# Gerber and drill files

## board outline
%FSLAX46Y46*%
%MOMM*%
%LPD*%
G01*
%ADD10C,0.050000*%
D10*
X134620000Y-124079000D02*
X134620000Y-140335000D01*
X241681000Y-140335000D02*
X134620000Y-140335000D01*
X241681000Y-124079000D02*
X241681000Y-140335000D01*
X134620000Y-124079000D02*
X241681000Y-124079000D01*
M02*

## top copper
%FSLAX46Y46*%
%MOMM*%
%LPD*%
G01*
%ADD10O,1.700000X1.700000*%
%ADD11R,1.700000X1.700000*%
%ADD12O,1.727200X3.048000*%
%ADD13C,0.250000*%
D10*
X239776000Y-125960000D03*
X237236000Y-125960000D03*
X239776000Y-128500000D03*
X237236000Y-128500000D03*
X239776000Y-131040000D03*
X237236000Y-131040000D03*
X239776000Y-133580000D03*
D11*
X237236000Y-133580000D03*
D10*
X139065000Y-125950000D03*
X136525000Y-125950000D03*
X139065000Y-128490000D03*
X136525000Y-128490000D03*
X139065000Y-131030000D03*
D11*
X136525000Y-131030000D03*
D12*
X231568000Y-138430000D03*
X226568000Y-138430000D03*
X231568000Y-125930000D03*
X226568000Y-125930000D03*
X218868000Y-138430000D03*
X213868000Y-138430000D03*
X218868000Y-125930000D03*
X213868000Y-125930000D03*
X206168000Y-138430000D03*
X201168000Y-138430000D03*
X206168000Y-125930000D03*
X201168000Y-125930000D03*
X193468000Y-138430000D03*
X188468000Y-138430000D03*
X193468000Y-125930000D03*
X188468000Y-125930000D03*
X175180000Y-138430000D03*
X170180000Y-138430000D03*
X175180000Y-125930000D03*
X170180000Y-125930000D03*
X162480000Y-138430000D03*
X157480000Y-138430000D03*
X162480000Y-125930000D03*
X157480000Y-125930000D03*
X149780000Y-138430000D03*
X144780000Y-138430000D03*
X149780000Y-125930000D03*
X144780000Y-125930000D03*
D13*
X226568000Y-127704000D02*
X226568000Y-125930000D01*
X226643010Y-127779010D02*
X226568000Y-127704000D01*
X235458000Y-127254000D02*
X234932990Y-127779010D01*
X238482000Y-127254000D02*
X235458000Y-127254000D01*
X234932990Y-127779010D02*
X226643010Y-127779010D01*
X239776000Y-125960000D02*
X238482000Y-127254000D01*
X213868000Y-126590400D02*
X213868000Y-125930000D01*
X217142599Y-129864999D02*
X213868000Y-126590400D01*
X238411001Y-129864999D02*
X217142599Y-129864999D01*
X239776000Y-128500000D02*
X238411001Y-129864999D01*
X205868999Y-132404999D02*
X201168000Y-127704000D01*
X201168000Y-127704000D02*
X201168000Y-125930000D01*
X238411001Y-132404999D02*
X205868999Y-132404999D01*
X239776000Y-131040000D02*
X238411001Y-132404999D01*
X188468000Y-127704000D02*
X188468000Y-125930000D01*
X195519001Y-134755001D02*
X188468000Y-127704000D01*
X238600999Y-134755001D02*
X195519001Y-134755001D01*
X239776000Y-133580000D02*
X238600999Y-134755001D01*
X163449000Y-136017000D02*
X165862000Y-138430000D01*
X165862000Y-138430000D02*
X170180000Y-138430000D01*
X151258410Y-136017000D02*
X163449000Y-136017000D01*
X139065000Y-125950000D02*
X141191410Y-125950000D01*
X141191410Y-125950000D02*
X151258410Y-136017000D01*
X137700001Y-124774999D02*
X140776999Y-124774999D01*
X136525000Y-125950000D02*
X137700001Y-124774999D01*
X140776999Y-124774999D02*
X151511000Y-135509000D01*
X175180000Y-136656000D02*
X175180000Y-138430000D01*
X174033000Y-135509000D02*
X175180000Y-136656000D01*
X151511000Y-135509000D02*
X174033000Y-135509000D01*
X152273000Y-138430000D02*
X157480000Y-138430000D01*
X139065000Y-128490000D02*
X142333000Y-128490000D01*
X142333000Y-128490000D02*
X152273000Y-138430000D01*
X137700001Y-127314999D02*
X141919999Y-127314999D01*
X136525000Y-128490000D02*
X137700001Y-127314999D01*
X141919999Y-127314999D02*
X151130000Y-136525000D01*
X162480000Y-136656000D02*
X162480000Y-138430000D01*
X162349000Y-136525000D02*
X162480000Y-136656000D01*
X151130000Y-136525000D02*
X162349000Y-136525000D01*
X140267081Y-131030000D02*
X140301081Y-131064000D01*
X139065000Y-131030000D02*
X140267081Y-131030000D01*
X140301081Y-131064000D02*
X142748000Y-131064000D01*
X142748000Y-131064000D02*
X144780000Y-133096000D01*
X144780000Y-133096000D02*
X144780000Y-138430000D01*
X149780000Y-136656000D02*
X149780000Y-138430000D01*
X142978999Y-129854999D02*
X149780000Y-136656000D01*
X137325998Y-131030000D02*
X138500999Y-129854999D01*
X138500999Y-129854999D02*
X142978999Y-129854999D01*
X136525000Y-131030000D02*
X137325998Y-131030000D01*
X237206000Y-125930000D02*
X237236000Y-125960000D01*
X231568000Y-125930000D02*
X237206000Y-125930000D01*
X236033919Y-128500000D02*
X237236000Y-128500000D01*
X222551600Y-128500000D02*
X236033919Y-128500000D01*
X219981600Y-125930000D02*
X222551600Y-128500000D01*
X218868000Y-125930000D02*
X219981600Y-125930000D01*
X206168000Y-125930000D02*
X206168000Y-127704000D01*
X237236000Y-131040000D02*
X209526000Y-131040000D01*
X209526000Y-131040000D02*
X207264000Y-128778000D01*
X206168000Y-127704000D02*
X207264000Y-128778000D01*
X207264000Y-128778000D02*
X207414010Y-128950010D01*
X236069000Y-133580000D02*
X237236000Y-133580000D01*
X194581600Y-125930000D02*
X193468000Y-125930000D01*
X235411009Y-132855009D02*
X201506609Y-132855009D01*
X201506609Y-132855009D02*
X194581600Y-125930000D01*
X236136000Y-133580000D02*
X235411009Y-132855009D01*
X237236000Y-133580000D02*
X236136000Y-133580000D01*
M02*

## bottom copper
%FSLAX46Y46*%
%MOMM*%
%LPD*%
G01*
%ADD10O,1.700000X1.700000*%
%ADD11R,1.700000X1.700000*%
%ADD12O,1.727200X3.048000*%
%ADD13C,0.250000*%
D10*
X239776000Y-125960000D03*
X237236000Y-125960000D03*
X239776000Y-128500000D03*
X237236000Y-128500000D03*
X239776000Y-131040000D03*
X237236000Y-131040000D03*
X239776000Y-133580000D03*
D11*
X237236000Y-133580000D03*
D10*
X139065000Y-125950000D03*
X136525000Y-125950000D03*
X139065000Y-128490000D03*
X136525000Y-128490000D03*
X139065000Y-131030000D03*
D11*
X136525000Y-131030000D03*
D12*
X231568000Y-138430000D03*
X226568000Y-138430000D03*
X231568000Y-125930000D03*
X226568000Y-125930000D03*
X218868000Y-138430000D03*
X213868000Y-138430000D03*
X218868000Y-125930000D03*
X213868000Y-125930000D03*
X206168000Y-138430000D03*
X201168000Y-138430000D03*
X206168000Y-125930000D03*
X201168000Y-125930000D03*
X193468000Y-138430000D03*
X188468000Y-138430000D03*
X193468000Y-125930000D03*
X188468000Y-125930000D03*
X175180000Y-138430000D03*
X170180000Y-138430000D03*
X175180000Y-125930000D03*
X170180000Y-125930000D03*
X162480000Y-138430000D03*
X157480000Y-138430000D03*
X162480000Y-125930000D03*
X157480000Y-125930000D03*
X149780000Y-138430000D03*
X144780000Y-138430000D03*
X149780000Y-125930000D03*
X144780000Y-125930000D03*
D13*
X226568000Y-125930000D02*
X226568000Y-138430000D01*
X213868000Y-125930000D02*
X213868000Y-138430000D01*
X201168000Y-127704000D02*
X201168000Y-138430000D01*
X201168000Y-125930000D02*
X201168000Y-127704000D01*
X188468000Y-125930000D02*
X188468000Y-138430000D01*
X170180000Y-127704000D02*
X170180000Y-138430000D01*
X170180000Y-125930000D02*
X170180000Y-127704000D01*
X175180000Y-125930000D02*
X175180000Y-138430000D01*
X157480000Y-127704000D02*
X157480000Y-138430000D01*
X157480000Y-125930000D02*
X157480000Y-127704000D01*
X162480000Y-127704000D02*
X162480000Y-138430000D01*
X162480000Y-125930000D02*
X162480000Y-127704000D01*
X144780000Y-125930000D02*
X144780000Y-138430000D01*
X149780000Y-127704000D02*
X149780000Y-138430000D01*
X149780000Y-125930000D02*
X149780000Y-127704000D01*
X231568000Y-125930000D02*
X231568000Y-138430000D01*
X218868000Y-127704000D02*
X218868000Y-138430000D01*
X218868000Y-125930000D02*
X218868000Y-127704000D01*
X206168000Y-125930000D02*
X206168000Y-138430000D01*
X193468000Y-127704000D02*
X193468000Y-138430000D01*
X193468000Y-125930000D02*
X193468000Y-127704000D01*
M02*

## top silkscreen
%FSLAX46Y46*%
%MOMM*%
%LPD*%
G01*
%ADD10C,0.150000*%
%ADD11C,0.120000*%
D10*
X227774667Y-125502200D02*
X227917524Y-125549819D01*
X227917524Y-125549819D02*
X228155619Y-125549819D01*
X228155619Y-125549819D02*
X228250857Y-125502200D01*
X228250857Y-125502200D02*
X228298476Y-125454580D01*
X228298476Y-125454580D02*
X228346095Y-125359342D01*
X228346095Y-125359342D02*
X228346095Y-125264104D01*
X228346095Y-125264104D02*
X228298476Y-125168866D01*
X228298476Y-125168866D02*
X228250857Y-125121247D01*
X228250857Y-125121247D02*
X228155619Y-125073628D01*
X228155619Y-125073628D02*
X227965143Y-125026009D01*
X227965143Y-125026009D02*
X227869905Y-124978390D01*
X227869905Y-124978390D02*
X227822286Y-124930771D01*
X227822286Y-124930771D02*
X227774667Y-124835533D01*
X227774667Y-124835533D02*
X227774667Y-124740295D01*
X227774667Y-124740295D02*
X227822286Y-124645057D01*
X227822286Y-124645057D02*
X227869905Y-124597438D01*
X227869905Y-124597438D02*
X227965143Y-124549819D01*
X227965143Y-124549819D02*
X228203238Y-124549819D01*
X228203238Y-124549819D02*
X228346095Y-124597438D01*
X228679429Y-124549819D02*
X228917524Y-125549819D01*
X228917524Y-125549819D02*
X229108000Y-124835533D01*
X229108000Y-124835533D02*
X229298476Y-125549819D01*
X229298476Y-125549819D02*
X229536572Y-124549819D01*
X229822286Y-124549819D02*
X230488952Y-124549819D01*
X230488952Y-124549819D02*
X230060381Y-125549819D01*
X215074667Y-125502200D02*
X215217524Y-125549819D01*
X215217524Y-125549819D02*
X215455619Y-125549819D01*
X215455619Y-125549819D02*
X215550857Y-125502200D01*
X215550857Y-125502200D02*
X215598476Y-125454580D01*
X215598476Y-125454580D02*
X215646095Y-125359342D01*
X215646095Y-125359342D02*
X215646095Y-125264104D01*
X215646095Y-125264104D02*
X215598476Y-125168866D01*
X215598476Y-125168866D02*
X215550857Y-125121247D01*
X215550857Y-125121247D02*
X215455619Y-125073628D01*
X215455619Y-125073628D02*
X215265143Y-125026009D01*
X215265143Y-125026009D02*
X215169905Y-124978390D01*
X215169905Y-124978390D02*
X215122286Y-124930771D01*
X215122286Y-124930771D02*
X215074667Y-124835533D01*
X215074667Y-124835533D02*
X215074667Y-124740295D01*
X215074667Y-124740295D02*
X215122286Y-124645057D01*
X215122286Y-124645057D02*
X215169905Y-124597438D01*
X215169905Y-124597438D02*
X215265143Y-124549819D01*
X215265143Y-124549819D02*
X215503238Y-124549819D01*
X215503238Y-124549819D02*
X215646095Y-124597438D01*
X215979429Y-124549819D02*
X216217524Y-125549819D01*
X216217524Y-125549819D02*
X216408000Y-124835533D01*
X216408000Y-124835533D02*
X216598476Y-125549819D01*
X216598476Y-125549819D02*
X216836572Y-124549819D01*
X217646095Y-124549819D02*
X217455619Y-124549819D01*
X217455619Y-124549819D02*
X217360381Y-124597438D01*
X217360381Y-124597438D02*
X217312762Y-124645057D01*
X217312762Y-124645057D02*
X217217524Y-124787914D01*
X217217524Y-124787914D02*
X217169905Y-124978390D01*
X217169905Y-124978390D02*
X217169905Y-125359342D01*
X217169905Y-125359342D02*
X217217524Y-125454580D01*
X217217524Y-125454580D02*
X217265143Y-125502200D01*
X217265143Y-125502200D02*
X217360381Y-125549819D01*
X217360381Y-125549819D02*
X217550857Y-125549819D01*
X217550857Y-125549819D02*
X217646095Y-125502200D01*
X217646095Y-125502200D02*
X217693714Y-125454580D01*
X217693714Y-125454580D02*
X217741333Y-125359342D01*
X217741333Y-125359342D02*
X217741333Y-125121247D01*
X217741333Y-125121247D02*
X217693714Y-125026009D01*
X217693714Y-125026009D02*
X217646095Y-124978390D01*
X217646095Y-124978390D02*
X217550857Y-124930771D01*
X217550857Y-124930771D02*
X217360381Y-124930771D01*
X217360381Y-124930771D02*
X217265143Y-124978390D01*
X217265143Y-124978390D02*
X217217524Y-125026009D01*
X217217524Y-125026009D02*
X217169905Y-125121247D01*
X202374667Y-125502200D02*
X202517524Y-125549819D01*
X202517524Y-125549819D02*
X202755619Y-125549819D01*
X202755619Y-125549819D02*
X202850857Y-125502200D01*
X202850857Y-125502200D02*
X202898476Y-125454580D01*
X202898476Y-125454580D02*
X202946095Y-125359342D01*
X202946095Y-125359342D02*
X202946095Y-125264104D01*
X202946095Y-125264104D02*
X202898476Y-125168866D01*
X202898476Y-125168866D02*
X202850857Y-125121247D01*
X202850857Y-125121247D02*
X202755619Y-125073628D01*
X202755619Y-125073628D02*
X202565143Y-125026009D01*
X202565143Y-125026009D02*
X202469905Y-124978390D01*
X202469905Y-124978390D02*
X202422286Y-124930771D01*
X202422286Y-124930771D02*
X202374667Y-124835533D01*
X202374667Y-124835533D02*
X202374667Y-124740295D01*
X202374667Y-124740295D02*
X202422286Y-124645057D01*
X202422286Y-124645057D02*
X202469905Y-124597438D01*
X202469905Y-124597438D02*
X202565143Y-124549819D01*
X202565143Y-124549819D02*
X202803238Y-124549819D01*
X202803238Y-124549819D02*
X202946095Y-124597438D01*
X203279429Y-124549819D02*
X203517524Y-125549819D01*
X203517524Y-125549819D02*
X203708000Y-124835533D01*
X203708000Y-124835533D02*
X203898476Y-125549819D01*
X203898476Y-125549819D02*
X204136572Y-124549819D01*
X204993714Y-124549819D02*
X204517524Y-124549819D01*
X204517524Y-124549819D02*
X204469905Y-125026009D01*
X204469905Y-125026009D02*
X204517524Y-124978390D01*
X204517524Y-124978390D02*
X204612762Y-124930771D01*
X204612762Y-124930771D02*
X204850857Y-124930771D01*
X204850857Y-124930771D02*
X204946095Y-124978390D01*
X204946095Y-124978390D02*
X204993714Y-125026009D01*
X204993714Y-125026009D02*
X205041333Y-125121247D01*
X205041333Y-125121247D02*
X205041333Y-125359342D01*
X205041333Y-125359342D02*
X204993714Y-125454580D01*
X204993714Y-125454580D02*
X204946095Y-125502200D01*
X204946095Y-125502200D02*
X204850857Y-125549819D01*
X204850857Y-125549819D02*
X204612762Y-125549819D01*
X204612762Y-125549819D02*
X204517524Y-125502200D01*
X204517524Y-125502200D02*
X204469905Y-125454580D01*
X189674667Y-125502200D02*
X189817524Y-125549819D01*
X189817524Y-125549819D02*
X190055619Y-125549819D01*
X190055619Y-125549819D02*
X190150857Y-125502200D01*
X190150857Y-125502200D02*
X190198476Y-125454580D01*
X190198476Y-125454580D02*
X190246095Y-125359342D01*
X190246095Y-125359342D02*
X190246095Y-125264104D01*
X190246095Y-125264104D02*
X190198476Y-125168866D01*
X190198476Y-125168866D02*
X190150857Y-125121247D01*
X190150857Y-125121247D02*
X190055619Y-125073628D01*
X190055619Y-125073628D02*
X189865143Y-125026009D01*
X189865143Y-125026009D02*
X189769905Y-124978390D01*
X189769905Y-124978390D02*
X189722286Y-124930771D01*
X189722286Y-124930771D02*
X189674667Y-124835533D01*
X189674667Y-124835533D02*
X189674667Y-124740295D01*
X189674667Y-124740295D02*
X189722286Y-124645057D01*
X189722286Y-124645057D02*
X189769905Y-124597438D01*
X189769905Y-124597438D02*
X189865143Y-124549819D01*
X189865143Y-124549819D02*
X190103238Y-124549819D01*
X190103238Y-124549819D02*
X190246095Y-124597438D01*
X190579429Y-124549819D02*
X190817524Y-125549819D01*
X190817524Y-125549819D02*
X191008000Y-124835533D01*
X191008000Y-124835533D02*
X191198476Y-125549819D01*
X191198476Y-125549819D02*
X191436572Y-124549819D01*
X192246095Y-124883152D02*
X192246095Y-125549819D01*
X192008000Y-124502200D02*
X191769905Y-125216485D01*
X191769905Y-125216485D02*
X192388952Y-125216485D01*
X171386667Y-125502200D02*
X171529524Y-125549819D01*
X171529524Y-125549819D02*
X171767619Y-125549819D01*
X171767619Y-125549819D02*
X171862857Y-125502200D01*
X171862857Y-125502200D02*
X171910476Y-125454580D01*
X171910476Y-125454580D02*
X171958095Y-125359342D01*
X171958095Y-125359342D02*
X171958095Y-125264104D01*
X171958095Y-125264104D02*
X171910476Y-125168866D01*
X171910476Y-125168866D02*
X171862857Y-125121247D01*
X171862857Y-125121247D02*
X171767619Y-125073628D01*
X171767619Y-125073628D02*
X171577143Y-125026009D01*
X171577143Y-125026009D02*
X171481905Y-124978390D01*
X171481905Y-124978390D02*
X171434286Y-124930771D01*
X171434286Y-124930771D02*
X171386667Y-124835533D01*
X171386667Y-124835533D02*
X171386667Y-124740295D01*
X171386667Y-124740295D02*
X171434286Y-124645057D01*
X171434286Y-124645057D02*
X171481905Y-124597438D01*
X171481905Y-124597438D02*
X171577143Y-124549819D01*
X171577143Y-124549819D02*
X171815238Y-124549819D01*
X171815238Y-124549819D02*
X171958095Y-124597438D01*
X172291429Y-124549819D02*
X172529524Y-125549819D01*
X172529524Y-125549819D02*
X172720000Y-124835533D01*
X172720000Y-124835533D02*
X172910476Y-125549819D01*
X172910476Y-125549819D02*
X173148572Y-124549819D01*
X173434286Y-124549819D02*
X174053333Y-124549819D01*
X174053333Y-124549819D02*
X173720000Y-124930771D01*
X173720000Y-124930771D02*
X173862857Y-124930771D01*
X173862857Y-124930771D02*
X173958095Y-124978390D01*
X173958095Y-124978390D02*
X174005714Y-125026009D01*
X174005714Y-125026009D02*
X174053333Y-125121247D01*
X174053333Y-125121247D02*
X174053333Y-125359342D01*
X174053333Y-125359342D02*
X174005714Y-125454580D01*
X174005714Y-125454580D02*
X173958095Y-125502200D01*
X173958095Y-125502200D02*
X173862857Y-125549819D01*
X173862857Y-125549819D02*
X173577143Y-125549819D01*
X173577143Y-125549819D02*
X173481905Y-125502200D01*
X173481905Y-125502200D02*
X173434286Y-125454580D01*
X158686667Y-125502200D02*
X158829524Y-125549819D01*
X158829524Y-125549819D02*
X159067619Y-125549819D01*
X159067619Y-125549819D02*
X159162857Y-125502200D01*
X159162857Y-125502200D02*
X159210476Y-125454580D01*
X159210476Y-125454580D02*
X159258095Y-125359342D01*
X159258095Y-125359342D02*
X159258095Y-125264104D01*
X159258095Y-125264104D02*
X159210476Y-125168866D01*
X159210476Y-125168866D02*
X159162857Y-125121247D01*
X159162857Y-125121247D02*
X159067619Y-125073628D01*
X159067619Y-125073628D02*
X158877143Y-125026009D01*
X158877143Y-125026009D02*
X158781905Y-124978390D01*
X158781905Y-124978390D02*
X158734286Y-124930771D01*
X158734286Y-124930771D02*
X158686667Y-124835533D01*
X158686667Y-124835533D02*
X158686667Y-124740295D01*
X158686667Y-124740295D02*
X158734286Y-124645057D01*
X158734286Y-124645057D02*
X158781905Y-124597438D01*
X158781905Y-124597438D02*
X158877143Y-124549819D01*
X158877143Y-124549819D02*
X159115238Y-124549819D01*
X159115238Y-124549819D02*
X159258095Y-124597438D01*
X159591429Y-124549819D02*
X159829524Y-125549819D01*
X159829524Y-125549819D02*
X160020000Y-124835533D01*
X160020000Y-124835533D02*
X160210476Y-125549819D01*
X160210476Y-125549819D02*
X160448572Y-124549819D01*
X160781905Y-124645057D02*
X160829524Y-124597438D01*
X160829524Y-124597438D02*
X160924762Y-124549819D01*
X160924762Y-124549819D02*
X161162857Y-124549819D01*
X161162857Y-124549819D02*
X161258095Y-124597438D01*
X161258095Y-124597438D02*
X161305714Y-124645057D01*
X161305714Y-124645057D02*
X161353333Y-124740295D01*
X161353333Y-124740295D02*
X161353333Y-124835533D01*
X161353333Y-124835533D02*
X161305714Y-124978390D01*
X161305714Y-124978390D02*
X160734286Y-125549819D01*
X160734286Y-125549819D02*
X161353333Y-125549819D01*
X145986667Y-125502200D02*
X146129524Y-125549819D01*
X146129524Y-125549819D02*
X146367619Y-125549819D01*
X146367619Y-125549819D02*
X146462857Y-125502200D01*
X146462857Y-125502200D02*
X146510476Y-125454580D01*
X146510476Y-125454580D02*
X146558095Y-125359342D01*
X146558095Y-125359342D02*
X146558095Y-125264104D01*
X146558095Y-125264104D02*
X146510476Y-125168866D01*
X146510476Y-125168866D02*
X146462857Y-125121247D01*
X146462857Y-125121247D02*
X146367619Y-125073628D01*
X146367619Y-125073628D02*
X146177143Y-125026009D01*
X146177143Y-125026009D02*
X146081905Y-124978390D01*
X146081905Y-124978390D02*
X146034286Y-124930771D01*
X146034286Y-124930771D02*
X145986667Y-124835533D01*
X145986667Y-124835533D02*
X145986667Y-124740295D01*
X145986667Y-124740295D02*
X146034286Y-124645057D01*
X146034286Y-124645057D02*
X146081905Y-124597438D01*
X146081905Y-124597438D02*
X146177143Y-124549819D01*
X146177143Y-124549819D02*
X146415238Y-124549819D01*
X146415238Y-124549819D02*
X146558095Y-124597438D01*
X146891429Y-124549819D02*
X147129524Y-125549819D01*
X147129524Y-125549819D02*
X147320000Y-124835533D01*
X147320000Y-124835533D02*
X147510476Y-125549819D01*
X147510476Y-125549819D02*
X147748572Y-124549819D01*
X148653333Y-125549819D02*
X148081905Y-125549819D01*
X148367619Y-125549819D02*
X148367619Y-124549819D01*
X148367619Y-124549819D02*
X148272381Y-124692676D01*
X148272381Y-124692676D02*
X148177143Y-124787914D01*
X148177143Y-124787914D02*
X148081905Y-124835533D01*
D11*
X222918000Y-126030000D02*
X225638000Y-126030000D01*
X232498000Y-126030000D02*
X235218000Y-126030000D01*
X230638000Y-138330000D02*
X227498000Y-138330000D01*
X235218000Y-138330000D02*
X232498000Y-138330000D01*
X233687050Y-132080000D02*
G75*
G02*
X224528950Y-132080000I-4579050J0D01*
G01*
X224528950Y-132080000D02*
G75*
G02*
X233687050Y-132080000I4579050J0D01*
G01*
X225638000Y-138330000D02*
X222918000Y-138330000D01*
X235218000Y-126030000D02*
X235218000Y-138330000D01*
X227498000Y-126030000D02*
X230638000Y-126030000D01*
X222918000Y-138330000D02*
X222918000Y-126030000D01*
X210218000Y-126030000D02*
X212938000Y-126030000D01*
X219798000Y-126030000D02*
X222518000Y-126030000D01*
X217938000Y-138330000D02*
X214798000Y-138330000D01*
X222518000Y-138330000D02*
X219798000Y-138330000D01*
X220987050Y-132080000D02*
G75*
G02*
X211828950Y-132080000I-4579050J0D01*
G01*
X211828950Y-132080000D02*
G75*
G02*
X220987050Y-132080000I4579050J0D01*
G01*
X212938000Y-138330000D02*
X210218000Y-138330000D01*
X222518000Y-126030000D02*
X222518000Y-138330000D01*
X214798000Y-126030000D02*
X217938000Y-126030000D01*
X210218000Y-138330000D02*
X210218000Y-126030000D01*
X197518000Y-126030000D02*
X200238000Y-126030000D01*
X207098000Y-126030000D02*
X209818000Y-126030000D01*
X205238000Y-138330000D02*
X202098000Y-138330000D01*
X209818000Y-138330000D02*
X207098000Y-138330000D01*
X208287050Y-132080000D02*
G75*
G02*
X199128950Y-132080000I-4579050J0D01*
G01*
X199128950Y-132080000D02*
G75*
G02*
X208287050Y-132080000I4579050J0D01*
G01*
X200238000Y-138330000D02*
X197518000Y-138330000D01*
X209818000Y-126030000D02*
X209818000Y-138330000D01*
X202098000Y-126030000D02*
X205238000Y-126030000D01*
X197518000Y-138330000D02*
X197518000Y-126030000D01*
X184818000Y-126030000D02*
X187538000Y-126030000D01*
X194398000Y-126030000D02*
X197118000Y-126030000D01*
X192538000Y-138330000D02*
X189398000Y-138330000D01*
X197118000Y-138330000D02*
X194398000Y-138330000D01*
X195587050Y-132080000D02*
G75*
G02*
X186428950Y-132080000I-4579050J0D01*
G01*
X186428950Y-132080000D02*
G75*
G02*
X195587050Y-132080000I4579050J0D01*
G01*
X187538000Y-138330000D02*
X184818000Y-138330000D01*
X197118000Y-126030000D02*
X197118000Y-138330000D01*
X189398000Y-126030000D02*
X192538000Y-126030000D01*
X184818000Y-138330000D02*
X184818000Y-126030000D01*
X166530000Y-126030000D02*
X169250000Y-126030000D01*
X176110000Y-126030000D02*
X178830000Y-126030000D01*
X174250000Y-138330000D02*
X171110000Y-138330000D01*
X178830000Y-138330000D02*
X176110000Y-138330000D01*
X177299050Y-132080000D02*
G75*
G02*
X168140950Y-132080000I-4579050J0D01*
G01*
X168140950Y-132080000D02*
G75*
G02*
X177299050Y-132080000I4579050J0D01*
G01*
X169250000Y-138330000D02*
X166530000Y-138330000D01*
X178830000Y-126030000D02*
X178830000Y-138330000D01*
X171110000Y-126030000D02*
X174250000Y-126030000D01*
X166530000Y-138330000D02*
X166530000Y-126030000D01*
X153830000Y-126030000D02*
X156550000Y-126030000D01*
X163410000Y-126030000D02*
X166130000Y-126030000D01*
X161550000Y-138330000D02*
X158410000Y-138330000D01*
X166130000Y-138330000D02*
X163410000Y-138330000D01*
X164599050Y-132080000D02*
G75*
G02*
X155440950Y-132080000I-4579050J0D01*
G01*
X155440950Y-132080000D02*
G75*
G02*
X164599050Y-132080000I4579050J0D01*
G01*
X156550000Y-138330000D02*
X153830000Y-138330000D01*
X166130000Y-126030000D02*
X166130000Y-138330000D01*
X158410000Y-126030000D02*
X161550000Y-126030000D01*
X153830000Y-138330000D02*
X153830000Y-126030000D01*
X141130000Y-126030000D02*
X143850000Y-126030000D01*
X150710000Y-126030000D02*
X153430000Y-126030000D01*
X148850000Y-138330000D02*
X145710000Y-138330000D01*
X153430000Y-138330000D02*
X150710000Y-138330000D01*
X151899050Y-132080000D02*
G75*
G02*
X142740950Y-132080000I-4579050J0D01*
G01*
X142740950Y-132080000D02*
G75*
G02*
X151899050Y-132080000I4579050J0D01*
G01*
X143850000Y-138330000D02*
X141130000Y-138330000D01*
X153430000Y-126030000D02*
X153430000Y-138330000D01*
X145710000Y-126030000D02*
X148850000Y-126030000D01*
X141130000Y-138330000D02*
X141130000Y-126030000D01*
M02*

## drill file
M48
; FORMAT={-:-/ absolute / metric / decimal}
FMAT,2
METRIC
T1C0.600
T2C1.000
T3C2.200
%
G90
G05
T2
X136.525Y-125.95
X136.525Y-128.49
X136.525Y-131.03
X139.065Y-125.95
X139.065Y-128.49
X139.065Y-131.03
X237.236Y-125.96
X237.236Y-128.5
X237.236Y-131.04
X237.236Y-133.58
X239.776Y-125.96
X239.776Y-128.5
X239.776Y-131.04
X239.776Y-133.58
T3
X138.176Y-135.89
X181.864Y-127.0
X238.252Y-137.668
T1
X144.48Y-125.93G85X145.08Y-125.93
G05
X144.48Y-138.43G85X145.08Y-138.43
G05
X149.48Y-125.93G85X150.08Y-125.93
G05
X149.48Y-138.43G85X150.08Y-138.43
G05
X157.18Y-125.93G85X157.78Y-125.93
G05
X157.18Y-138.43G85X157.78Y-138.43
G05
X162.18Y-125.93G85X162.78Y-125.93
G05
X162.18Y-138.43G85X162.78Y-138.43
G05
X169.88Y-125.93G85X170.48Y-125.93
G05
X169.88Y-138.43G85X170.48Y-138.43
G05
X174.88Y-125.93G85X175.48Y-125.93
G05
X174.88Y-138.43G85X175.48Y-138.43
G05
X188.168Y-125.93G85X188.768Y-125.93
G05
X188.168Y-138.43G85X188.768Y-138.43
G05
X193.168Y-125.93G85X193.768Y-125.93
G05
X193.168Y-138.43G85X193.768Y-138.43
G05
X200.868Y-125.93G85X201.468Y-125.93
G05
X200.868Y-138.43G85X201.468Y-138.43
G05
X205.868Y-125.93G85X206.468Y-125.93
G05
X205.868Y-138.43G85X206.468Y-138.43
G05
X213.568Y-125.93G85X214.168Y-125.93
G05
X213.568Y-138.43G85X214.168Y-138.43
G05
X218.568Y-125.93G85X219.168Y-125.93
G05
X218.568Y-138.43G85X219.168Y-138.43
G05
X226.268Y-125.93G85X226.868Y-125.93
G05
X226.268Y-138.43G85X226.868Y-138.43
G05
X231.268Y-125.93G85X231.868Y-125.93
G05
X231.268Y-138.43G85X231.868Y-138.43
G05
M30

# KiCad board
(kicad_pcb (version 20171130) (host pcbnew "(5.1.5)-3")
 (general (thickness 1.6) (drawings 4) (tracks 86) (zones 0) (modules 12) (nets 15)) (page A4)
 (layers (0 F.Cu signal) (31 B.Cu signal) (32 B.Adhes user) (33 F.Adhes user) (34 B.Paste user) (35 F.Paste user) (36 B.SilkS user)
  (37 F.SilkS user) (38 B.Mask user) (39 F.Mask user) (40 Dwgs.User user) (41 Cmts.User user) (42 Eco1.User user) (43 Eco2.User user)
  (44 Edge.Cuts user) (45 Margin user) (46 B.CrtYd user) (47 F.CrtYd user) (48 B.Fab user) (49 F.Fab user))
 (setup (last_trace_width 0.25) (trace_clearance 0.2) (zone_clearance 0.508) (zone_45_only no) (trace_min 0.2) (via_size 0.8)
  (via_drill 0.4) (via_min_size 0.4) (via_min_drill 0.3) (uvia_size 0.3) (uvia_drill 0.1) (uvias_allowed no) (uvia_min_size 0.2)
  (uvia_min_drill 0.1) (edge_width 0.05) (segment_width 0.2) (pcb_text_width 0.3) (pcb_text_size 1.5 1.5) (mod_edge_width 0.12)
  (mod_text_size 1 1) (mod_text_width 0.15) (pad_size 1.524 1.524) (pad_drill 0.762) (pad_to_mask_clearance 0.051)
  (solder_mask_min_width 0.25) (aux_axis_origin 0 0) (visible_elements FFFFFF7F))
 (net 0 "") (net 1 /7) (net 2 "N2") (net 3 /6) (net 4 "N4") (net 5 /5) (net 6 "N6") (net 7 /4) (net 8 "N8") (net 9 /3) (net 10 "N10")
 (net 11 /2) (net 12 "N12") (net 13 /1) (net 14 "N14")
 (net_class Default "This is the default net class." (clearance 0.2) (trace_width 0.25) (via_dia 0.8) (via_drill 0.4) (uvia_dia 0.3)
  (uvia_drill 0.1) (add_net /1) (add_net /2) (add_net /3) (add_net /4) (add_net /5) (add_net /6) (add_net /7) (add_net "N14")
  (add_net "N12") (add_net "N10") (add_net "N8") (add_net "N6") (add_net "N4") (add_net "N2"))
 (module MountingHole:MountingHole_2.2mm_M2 (layer F.Cu) (at 181.864 127)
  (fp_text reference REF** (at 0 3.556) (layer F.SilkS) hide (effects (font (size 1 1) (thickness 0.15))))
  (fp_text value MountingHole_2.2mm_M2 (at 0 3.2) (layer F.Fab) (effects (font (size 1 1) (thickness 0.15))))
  (pad 1 np_thru_hole circle (at 0 0) (size 2.2 2.2) (drill 2.2) (layers *.Cu *.Mask)))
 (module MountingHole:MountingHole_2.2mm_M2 (layer F.Cu) (at 238.252 137.668)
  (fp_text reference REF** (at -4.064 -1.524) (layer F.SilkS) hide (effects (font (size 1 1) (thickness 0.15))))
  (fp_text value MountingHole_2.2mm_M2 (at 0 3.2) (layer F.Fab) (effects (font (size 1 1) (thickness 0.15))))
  (pad 1 np_thru_hole circle (at 0 0) (size 2.2 2.2) (drill 2.2) (layers *.Cu *.Mask)))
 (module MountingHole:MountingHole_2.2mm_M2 (layer F.Cu) (at 138.176 135.89)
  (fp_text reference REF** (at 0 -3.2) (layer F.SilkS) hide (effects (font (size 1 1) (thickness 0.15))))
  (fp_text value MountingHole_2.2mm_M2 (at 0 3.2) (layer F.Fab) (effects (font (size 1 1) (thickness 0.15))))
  (pad 1 np_thru_hole circle (at 0 0) (size 2.2 2.2) (drill 2.2) (layers *.Cu *.Mask)))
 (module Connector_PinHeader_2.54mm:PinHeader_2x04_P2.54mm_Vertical (layer B.Cu) (at 237.236 133.58)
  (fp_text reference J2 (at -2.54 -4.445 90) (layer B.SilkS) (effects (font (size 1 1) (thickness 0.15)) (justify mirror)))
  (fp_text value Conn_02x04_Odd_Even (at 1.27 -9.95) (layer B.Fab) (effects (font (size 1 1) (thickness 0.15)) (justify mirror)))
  (pad 8 thru_hole oval (at 2.54 -7.62) (size 1.7 1.7) (drill 1) (layers *.Cu *.Mask) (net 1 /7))
  (pad 7 thru_hole oval (at 0 -7.62) (size 1.7 1.7) (drill 1) (layers *.Cu *.Mask) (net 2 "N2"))
  (pad 6 thru_hole oval (at 2.54 -5.08) (size 1.7 1.7) (drill 1) (layers *.Cu *.Mask) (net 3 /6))
  (pad 5 thru_hole oval (at 0 -5.08) (size 1.7 1.7) (drill 1) (layers *.Cu *.Mask) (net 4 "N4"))
  (pad 4 thru_hole oval (at 2.54 -2.54) (size 1.7 1.7) (drill 1) (layers *.Cu *.Mask) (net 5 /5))
  (pad 3 thru_hole oval (at 0 -2.54) (size 1.7 1.7) (drill 1) (layers *.Cu *.Mask) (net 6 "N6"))
  (pad 2 thru_hole oval (at 2.54 0) (size 1.7 1.7) (drill 1) (layers *.Cu *.Mask) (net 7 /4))
  (pad 1 thru_hole rect (at 0 0) (size 1.7 1.7) (drill 1) (layers *.Cu *.Mask) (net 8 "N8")))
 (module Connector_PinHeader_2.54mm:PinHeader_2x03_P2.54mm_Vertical (layer B.Cu) (at 136.525 131.03)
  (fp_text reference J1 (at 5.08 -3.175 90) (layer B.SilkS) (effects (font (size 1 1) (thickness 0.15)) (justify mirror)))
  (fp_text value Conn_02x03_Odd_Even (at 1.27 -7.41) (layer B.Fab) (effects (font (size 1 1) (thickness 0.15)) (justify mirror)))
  (pad 6 thru_hole oval (at 2.54 -5.08) (size 1.7 1.7) (drill 1) (layers *.Cu *.Mask) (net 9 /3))
  (pad 5 thru_hole oval (at 0 -5.08) (size 1.7 1.7) (drill 1) (layers *.Cu *.Mask) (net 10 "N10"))
  (pad 4 thru_hole oval (at 2.54 -2.54) (size 1.7 1.7) (drill 1) (layers *.Cu *.Mask) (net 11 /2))
  (pad 3 thru_hole oval (at 0 -2.54) (size 1.7 1.7) (drill 1) (layers *.Cu *.Mask) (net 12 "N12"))
  (pad 2 thru_hole oval (at 2.54 0) (size 1.7 1.7) (drill 1) (layers *.Cu *.Mask) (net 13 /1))
  (pad 1 thru_hole rect (at 0 0) (size 1.7 1.7) (drill 1) (layers *.Cu *.Mask) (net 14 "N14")))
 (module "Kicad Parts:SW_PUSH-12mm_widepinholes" (layer F.Cu) (at 226.568 138.43 90)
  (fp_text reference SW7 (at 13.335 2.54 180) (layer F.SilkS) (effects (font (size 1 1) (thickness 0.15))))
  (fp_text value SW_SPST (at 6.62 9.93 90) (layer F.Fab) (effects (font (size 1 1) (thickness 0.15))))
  (fp_line (start 12.4 -3.65) (end 12.4 -0.93) (layer F.SilkS) (width 0.12))
  (fp_line (start 12.4 5.93) (end 12.4 8.65) (layer F.SilkS) (width 0.12))
  (fp_line (start 0.1 4.07) (end 0.1 0.93) (layer F.SilkS) (width 0.12))
  (fp_line (start 0.1 8.65) (end 0.1 5.93) (layer F.SilkS) (width 0.12))
  (fp_circle (center 6.35 2.54) (end 10.16 5.08) (layer F.SilkS) (width 0.12))
  (fp_line (start 0.1 -0.93) (end 0.1 -3.65) (layer F.SilkS) (width 0.12))
  (fp_line (start 12.4 8.65) (end 0.1 8.65) (layer F.SilkS) (width 0.12))
  (fp_line (start 12.4 0.93) (end 12.4 4.07) (layer F.SilkS) (width 0.12))
  (fp_line (start 0.1 -3.65) (end 12.4 -3.65) (layer F.SilkS) (width 0.12))
  (pad 2 thru_hole oval (at 0 5 90) (size 3.048 1.7272) (drill oval 0.6 1.2) (layers *.Cu *.Mask) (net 2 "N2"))
  (pad 1 thru_hole oval (at 0 0 90) (size 3.048 1.7272) (drill oval 0.6 1.2) (layers *.Cu *.Mask) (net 1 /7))
  (pad 2 thru_hole oval (at 12.5 5 90) (size 3.048 1.7272) (drill oval 0.6 1.2) (layers *.Cu *.Mask) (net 2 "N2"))
  (pad 1 thru_hole oval (at 12.5 0 90) (size 3.048 1.7272) (drill oval 0.6 1.2) (layers *.Cu *.Mask) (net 1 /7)))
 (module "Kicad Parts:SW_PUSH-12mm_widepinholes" (layer F.Cu) (at 213.868 138.43 90)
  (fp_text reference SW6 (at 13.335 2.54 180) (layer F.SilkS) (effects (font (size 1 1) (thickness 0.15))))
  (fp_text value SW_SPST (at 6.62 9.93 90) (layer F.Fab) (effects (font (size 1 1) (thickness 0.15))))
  (fp_line (start 12.4 -3.65) (end 12.4 -0.93) (layer F.SilkS) (width 0.12))
  (fp_line (start 12.4 5.93) (end 12.4 8.65) (layer F.SilkS) (width 0.12))
  (fp_line (start 0.1 4.07) (end 0.1 0.93) (layer F.SilkS) (width 0.12))
  (fp_line (start 0.1 8.65) (end 0.1 5.93) (layer F.SilkS) (width 0.12))
  (fp_circle (center 6.35 2.54) (end 10.16 5.08) (layer F.SilkS) (width 0.12))
  (fp_line (start 0.1 -0.93) (end 0.1 -3.65) (layer F.SilkS) (width 0.12))
  (fp_line (start 12.4 8.65) (end 0.1 8.65) (layer F.SilkS) (width 0.12))
  (fp_line (start 12.4 0.93) (end 12.4 4.07) (layer F.SilkS) (width 0.12))
  (fp_line (start 0.1 -3.65) (end 12.4 -3.65) (layer F.SilkS) (width 0.12))
  (pad 2 thru_hole oval (at 0 5 90) (size 3.048 1.7272) (drill oval 0.6 1.2) (layers *.Cu *.Mask) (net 4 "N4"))
  (pad 1 thru_hole oval (at 0 0 90) (size 3.048 1.7272) (drill oval 0.6 1.2) (layers *.Cu *.Mask) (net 3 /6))
  (pad 2 thru_hole oval (at 12.5 5 90) (size 3.048 1.7272) (drill oval 0.6 1.2) (layers *.Cu *.Mask) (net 4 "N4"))
  (pad 1 thru_hole oval (at 12.5 0 90) (size 3.048 1.7272) (drill oval 0.6 1.2) (layers *.Cu *.Mask) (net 3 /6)))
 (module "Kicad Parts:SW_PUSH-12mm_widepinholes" (layer F.Cu) (at 201.168 138.43 90)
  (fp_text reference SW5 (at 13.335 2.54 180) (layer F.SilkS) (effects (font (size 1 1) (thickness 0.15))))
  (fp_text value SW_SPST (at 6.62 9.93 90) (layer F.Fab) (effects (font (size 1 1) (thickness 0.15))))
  (fp_line (start 12.4 -3.65) (end 12.4 -0.93) (layer F.SilkS) (width 0.12))
  (fp_line (start 12.4 5.93) (end 12.4 8.65) (layer F.SilkS) (width 0.12))
  (fp_line (start 0.1 4.07) (end 0.1 0.93) (layer F.SilkS) (width 0.12))
  (fp_line (start 0.1 8.65) (end 0.1 5.93) (layer F.SilkS) (width 0.12))
  (fp_circle (center 6.35 2.54) (end 10.16 5.08) (layer F.SilkS) (width 0.12))
  (fp_line (start 0.1 -0.93) (end 0.1 -3.65) (layer F.SilkS) (width 0.12))
  (fp_line (start 12.4 8.65) (end 0.1 8.65) (layer F.SilkS) (width 0.12))
  (fp_line (start 12.4 0.93) (end 12.4 4.07) (layer F.SilkS) (width 0.12))
  (fp_line (start 0.1 -3.65) (end 12.4 -3.65) (layer F.SilkS) (width 0.12))
  (pad 2 thru_hole oval (at 0 5 90) (size 3.048 1.7272) (drill oval 0.6 1.2) (layers *.Cu *.Mask) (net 6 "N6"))
  (pad 1 thru_hole oval (at 0 0 90) (size 3.048 1.7272) (drill oval 0.6 1.2) (layers *.Cu *.Mask) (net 5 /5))
  (pad 2 thru_hole oval (at 12.5 5 90) (size 3.048 1.7272) (drill oval 0.6 1.2) (layers *.Cu *.Mask) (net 6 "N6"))
  (pad 1 thru_hole oval (at 12.5 0 90) (size 3.048 1.7272) (drill oval 0.6 1.2) (layers *.Cu *.Mask) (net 5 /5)))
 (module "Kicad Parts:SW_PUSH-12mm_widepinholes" (layer F.Cu) (at 188.468 138.43 90)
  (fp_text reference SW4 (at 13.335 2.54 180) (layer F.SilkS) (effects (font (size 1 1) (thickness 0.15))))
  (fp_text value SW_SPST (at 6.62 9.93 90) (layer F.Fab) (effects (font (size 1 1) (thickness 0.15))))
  (fp_line (start 12.4 -3.65) (end 12.4 -0.93) (layer F.SilkS) (width 0.12))
  (fp_line (start 12.4 5.93) (end 12.4 8.65) (layer F.SilkS) (width 0.12))
  (fp_line (start 0.1 4.07) (end 0.1 0.93) (layer F.SilkS) (width 0.12))
  (fp_line (start 0.1 8.65) (end 0.1 5.93) (layer F.SilkS) (width 0.12))
  (fp_circle (center 6.35 2.54) (end 10.16 5.08) (layer F.SilkS) (width 0.12))
  (fp_line (start 0.1 -0.93) (end 0.1 -3.65) (layer F.SilkS) (width 0.12))
  (fp_line (start 12.4 8.65) (end 0.1 8.65) (layer F.SilkS) (width 0.12))
  (fp_line (start 12.4 0.93) (end 12.4 4.07) (layer F.SilkS) (width 0.12))
  (fp_line (start 0.1 -3.65) (end 12.4 -3.65) (layer F.SilkS) (width 0.12))
  (pad 2 thru_hole oval (at 0 5 90) (size 3.048 1.7272) (drill oval 0.6 1.2) (layers *.Cu *.Mask) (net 8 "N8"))
  (pad 1 thru_hole oval (at 0 0 90) (size 3.048 1.7272) (drill oval 0.6 1.2) (layers *.Cu *.Mask) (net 7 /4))
  (pad 2 thru_hole oval (at 12.5 5 90) (size 3.048 1.7272) (drill oval 0.6 1.2) (layers *.Cu *.Mask) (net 8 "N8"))
  (pad 1 thru_hole oval (at 12.5 0 90) (size 3.048 1.7272) (drill oval 0.6 1.2) (layers *.Cu *.Mask) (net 7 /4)))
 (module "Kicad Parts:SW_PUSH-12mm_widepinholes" (layer F.Cu) (at 170.18 138.43 90)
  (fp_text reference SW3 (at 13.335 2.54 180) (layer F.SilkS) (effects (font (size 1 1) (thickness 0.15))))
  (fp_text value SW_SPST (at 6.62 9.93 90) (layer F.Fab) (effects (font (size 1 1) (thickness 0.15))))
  (fp_line (start 12.4 -3.65) (end 12.4 -0.93) (layer F.SilkS) (width 0.12))
  (fp_line (start 12.4 5.93) (end 12.4 8.65) (layer F.SilkS) (width 0.12))
  (fp_line (start 0.1 4.07) (end 0.1 0.93) (layer F.SilkS) (width 0.12))
  (fp_line (start 0.1 8.65) (end 0.1 5.93) (layer F.SilkS) (width 0.12))
  (fp_circle (center 6.35 2.54) (end 10.16 5.08) (layer F.SilkS) (width 0.12))
  (fp_line (start 0.1 -0.93) (end 0.1 -3.65) (layer F.SilkS) (width 0.12))
  (fp_line (start 12.4 8.65) (end 0.1 8.65) (layer F.SilkS) (width 0.12))
  (fp_line (start 12.4 0.93) (end 12.4 4.07) (layer F.SilkS) (width 0.12))
  (fp_line (start 0.1 -3.65) (end 12.4 -3.65) (layer F.SilkS) (width 0.12))
  (pad 2 thru_hole oval (at 0 5 90) (size 3.048 1.7272) (drill oval 0.6 1.2) (layers *.Cu *.Mask) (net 10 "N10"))
  (pad 1 thru_hole oval (at 0 0 90) (size 3.048 1.7272) (drill oval 0.6 1.2) (layers *.Cu *.Mask) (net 9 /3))
  (pad 2 thru_hole oval (at 12.5 5 90) (size 3.048 1.7272) (drill oval 0.6 1.2) (layers *.Cu *.Mask) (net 10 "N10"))
  (pad 1 thru_hole oval (at 12.5 0 90) (size 3.048 1.7272) (drill oval 0.6 1.2) (layers *.Cu *.Mask) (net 9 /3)))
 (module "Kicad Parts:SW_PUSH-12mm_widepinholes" (layer F.Cu) (at 157.48 138.43 90)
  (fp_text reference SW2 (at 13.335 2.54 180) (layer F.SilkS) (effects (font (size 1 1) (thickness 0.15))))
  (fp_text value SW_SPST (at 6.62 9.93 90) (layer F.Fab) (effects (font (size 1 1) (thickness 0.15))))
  (fp_line (start 12.4 -3.65) (end 12.4 -0.93) (layer F.SilkS) (width 0.12))
  (fp_line (start 12.4 5.93) (end 12.4 8.65) (layer F.SilkS) (width 0.12))
  (fp_line (start 0.1 4.07) (end 0.1 0.93) (layer F.SilkS) (width 0.12))
  (fp_line (start 0.1 8.65) (end 0.1 5.93) (layer F.SilkS) (width 0.12))
  (fp_circle (center 6.35 2.54) (end 10.16 5.08) (layer F.SilkS) (width 0.12))
  (fp_line (start 0.1 -0.93) (end 0.1 -3.65) (layer F.SilkS) (width 0.12))
  (fp_line (start 12.4 8.65) (end 0.1 8.65) (layer F.SilkS) (width 0.12))
  (fp_line (start 12.4 0.93) (end 12.4 4.07) (layer F.SilkS) (width 0.12))
  (fp_line (start 0.1 -3.65) (end 12.4 -3.65) (layer F.SilkS) (width 0.12))
  (pad 2 thru_hole oval (at 0 5 90) (size 3.048 1.7272) (drill oval 0.6 1.2) (layers *.Cu *.Mask) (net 12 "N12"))
  (pad 1 thru_hole oval (at 0 0 90) (size 3.048 1.7272) (drill oval 0.6 1.2) (layers *.Cu *.Mask) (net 11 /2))
  (pad 2 thru_hole oval (at 12.5 5 90) (size 3.048 1.7272) (drill oval 0.6 1.2) (layers *.Cu *.Mask) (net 12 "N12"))
  (pad 1 thru_hole oval (at 12.5 0 90) (size 3.048 1.7272) (drill oval 0.6 1.2) (layers *.Cu *.Mask) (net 11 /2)))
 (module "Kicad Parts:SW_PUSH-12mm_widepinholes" (layer F.Cu) (at 144.78 138.43 90)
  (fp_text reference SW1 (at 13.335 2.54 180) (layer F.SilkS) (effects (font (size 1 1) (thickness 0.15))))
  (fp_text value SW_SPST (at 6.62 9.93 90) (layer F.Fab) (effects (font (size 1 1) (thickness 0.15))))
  (fp_line (start 12.4 -3.65) (end 12.4 -0.93) (layer F.SilkS) (width 0.12))
  (fp_line (start 12.4 5.93) (end 12.4 8.65) (layer F.SilkS) (width 0.12))
  (fp_line (start 0.1 4.07) (end 0.1 0.93) (layer F.SilkS) (width 0.12))
  (fp_line (start 0.1 8.65) (end 0.1 5.93) (layer F.SilkS) (width 0.12))
  (fp_circle (center 6.35 2.54) (end 10.16 5.08) (layer F.SilkS) (width 0.12))
  (fp_line (start 0.1 -0.93) (end 0.1 -3.65) (layer F.SilkS) (width 0.12))
  (fp_line (start 12.4 8.65) (end 0.1 8.65) (layer F.SilkS) (width 0.12))
  (fp_line (start 12.4 0.93) (end 12.4 4.07) (layer F.SilkS) (width 0.12))
  (fp_line (start 0.1 -3.65) (end 12.4 -3.65) (layer F.SilkS) (width 0.12))
  (pad 2 thru_hole oval (at 0 5 90) (size 3.048 1.7272) (drill oval 0.6 1.2) (layers *.Cu *.Mask) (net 14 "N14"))
  (pad 1 thru_hole oval (at 0 0 90) (size 3.048 1.7272) (drill oval 0.6 1.2) (layers *.Cu *.Mask) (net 13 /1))
  (pad 2 thru_hole oval (at 12.5 5 90) (size 3.048 1.7272) (drill oval 0.6 1.2) (layers *.Cu *.Mask) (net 14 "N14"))
  (pad 1 thru_hole oval (at 12.5 0 90) (size 3.048 1.7272) (drill oval 0.6 1.2) (layers *.Cu *.Mask) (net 13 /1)))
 (gr_line (start 134.62 124.079) (end 134.62 140.335) (layer Edge.Cuts) (width 0.05))
 (gr_line (start 241.681 140.335) (end 134.62 140.335) (layer Edge.Cuts) (width 0.05))
 (gr_line (start 241.681 124.079) (end 241.681 140.335) (layer Edge.Cuts) (width 0.05))
 (gr_line (start 134.62 124.079) (end 241.681 124.079) (layer Edge.Cuts) (width 0.05))
 (segment (start 226.568 125.93) (end 226.568 138.43) (width 0.25) (layer B.Cu) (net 1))
 (segment (start 226.568 127.704) (end 226.568 125.93) (width 0.25) (layer F.Cu) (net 1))
 (segment (start 226.64301 127.77901) (end 226.568 127.704) (width 0.25) (layer F.Cu) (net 1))
 (segment (start 235.458 127.254) (end 234.93299 127.77901) (width 0.25) (layer F.Cu) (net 1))
 (segment (start 238.482 127.254) (end 235.458 127.254) (width 0.25) (layer F.Cu) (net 1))
 (segment (start 234.93299 127.77901) (end 226.64301 127.77901) (width 0.25) (layer F.Cu) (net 1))
 (segment (start 239.776 125.96) (end 238.482 127.254) (width 0.25) (layer F.Cu) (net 1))
 (segment (start 213.868 125.93) (end 213.868 138.43) (width 0.25) (layer B.Cu) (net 3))
 (segment (start 213.868 126.5904) (end 213.868 125.93) (width 0.25) (layer F.Cu) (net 3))
 (segment (start 217.142599 129.864999) (end 213.868 126.5904) (width 0.25) (layer F.Cu) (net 3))
 (segment (start 238.411001 129.864999) (end 217.142599 129.864999) (width 0.25) (layer F.Cu) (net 3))
 (segment (start 239.776 128.5) (end 238.411001 129.864999) (width 0.25) (layer F.Cu) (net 3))
 (segment (start 201.168 127.704) (end 201.168 138.43) (width 0.25) (layer B.Cu) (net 5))
 (segment (start 201.168 125.93) (end 201.168 127.704) (width 0.25) (layer B.Cu) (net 5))
 (segment (start 205.868999 132.404999) (end 201.168 127.704) (width 0.25) (layer F.Cu) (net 5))
 (segment (start 201.168 127.704) (end 201.168 125.93) (width 0.25) (layer F.Cu) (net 5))
 (segment (start 238.411001 132.404999) (end 205.868999 132.404999) (width 0.25) (layer F.Cu) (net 5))
 (segment (start 239.776 131.04) (end 238.411001 132.404999) (width 0.25) (layer F.Cu) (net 5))
 (segment (start 188.468 125.93) (end 188.468 138.43) (width 0.25) (layer B.Cu) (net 7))
 (segment (start 188.468 127.704) (end 188.468 125.93) (width 0.25) (layer F.Cu) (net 7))
 (segment (start 195.519001 134.755001) (end 188.468 127.704) (width 0.25) (layer F.Cu) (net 7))
 (segment (start 238.600999 134.755001) (end 195.519001 134.755001) (width 0.25) (layer F.Cu) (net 7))
 (segment (start 239.776 133.58) (end 238.600999 134.755001) (width 0.25) (layer F.Cu) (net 7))
 (segment (start 170.18 127.704) (end 170.18 138.43) (width 0.25) (layer B.Cu) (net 9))
 (segment (start 170.18 125.93) (end 170.18 127.704) (width 0.25) (layer B.Cu) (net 9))
 (segment (start 163.449 136.017) (end 165.862 138.43) (width 0.25) (layer F.Cu) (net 9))
 (segment (start 165.862 138.43) (end 170.18 138.43) (width 0.25) (layer F.Cu) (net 9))
 (segment (start 151.25841 136.017) (end 163.449 136.017) (width 0.25) (layer F.Cu) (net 9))
 (segment (start 139.065 125.95) (end 141.19141 125.95) (width 0.25) (layer F.Cu) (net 9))
 (segment (start 141.19141 125.95) (end 151.25841 136.017) (width 0.25) (layer F.Cu) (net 9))
 (segment (start 175.18 125.93) (end 175.18 138.43) (width 0.25) (layer B.Cu) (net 10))
 (segment (start 137.700001 124.774999) (end 140.776999 124.774999) (width 0.25) (layer F.Cu) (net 10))
 (segment (start 136.525 125.95) (end 137.700001 124.774999) (width 0.25) (layer F.Cu) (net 10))
 (segment (start 140.776999 124.774999) (end 151.511 135.509) (width 0.25) (layer F.Cu) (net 10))
 (segment (start 175.18 136.656) (end 175.18 138.43) (width 0.25) (layer F.Cu) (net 10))
 (segment (start 174.033 135.509) (end 175.18 136.656) (width 0.25) (layer F.Cu) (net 10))
 (segment (start 151.511 135.509) (end 174.033 135.509) (width 0.25) (layer F.Cu) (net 10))
 (segment (start 157.48 127.704) (end 157.48 138.43) (width 0.25) (layer B.Cu) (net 11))
 (segment (start 157.48 125.93) (end 157.48 127.704) (width 0.25) (layer B.Cu) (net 11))
 (segment (start 152.273 138.43) (end 157.48 138.43) (width 0.25) (layer F.Cu) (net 11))
 (segment (start 139.065 128.49) (end 142.333 128.49) (width 0.25) (layer F.Cu) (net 11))
 (segment (start 142.333 128.49) (end 152.273 138.43) (width 0.25) (layer F.Cu) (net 11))
 (segment (start 162.48 127.704) (end 162.48 138.43) (width 0.25) (layer B.Cu) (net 12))
 (segment (start 162.48 125.93) (end 162.48 127.704) (width 0.25) (layer B.Cu) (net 12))
 (segment (start 137.700001 127.314999) (end 141.919999 127.314999) (width 0.25) (layer F.Cu) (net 12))
 (segment (start 136.525 128.49) (end 137.700001 127.314999) (width 0.25) (layer F.Cu) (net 12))
 (segment (start 141.919999 127.314999) (end 151.13 136.525) (width 0.25) (layer F.Cu) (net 12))
 (segment (start 162.48 136.656) (end 162.48 138.43) (width 0.25) (layer F.Cu) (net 12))
 (segment (start 162.349 136.525) (end 162.48 136.656) (width 0.25) (layer F.Cu) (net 12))
 (segment (start 151.13 136.525) (end 162.349 136.525) (width 0.25) (layer F.Cu) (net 12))
 (segment (start 144.78 125.93) (end 144.78 138.43) (width 0.25) (layer B.Cu) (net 13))
 (segment (start 140.267081 131.03) (end 140.301081 131.064) (width 0.25) (layer F.Cu) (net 13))
 (segment (start 139.065 131.03) (end 140.267081 131.03) (width 0.25) (layer F.Cu) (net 13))
 (segment (start 140.301081 131.064) (end 142.748 131.064) (width 0.25) (layer F.Cu) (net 13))
 (segment (start 142.748 131.064) (end 144.78 133.096) (width 0.25) (layer F.Cu) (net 13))
 (segment (start 144.78 133.096) (end 144.78 138.43) (width 0.25) (layer F.Cu) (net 13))
 (segment (start 149.78 127.704) (end 149.78 138.43) (width 0.25) (layer B.Cu) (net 14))
 (segment (start 149.78 125.93) (end 149.78 127.704) (width 0.25) (layer B.Cu) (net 14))
 (segment (start 149.78 136.656) (end 149.78 138.43) (width 0.25) (layer F.Cu) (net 14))
 (segment (start 142.978999 129.854999) (end 149.78 136.656) (width 0.25) (layer F.Cu) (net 14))
 (segment (start 137.325998 131.03) (end 138.500999 129.854999) (width 0.25) (layer F.Cu) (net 14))
 (segment (start 138.500999 129.854999) (end 142.978999 129.854999) (width 0.25) (layer F.Cu) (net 14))
 (segment (start 136.525 131.03) (end 137.325998 131.03) (width 0.25) (layer F.Cu) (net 14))
 (segment (start 231.568 125.93) (end 231.568 138.43) (width 0.25) (layer B.Cu) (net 2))
 (segment (start 237.206 125.93) (end 237.236 125.96) (width 0.25) (layer F.Cu) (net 2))
 (segment (start 231.568 125.93) (end 237.206 125.93) (width 0.25) (layer F.Cu) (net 2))
 (segment (start 218.868 127.704) (end 218.868 138.43) (width 0.25) (layer B.Cu) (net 4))
 (segment (start 218.868 125.93) (end 218.868 127.704) (width 0.25) (layer B.Cu) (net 4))
 (segment (start 236.033919 128.5) (end 237.236 128.5) (width 0.25) (layer F.Cu) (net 4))
 (segment (start 222.5516 128.5) (end 236.033919 128.5) (width 0.25) (layer F.Cu) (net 4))
 (segment (start 219.9816 125.93) (end 222.5516 128.5) (width 0.25) (layer F.Cu) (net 4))
 (segment (start 218.868 125.93) (end 219.9816 125.93) (width 0.25) (layer F.Cu) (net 4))
 (segment (start 206.168 125.93) (end 206.168 138.43) (width 0.25) (layer B.Cu) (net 6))
 (segment (start 206.168 125.93) (end 206.168 127.704) (width 0.25) (layer F.Cu) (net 6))
 (segment (start 237.236 131.04) (end 209.526 131.04) (width 0.25) (layer F.Cu) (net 6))
 (segment (start 209.526 131.04) (end 207.264 128.778) (width 0.25) (layer F.Cu) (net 6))
 (segment (start 206.168 127.704) (end 207.264 128.778) (width 0.25) (layer F.Cu) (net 6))
 (segment (start 207.264 128.778) (end 207.41401 128.95001) (width 0.25) (layer F.Cu) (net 6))
 (segment (start 193.468 127.704) (end 193.468 138.43) (width 0.25) (layer B.Cu) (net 8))
 (segment (start 193.468 125.93) (end 193.468 127.704) (width 0.25) (layer B.Cu) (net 8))
 (segment (start 236.069 133.58) (end 237.236 133.58) (width 0.25) (layer F.Cu) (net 8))
 (segment (start 194.5816 125.93) (end 193.468 125.93) (width 0.25) (layer F.Cu) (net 8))
 (segment (start 235.411009 132.855009) (end 201.506609 132.855009) (width 0.25) (layer F.Cu) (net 8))
 (segment (start 201.506609 132.855009) (end 194.5816 125.93) (width 0.25) (layer F.Cu) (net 8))
 (segment (start 236.136 133.58) (end 235.411009 132.855009) (width 0.25) (layer F.Cu) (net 8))
 (segment (start 237.236 133.58) (end 236.136 133.58) (width 0.25) (layer F.Cu) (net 8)))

